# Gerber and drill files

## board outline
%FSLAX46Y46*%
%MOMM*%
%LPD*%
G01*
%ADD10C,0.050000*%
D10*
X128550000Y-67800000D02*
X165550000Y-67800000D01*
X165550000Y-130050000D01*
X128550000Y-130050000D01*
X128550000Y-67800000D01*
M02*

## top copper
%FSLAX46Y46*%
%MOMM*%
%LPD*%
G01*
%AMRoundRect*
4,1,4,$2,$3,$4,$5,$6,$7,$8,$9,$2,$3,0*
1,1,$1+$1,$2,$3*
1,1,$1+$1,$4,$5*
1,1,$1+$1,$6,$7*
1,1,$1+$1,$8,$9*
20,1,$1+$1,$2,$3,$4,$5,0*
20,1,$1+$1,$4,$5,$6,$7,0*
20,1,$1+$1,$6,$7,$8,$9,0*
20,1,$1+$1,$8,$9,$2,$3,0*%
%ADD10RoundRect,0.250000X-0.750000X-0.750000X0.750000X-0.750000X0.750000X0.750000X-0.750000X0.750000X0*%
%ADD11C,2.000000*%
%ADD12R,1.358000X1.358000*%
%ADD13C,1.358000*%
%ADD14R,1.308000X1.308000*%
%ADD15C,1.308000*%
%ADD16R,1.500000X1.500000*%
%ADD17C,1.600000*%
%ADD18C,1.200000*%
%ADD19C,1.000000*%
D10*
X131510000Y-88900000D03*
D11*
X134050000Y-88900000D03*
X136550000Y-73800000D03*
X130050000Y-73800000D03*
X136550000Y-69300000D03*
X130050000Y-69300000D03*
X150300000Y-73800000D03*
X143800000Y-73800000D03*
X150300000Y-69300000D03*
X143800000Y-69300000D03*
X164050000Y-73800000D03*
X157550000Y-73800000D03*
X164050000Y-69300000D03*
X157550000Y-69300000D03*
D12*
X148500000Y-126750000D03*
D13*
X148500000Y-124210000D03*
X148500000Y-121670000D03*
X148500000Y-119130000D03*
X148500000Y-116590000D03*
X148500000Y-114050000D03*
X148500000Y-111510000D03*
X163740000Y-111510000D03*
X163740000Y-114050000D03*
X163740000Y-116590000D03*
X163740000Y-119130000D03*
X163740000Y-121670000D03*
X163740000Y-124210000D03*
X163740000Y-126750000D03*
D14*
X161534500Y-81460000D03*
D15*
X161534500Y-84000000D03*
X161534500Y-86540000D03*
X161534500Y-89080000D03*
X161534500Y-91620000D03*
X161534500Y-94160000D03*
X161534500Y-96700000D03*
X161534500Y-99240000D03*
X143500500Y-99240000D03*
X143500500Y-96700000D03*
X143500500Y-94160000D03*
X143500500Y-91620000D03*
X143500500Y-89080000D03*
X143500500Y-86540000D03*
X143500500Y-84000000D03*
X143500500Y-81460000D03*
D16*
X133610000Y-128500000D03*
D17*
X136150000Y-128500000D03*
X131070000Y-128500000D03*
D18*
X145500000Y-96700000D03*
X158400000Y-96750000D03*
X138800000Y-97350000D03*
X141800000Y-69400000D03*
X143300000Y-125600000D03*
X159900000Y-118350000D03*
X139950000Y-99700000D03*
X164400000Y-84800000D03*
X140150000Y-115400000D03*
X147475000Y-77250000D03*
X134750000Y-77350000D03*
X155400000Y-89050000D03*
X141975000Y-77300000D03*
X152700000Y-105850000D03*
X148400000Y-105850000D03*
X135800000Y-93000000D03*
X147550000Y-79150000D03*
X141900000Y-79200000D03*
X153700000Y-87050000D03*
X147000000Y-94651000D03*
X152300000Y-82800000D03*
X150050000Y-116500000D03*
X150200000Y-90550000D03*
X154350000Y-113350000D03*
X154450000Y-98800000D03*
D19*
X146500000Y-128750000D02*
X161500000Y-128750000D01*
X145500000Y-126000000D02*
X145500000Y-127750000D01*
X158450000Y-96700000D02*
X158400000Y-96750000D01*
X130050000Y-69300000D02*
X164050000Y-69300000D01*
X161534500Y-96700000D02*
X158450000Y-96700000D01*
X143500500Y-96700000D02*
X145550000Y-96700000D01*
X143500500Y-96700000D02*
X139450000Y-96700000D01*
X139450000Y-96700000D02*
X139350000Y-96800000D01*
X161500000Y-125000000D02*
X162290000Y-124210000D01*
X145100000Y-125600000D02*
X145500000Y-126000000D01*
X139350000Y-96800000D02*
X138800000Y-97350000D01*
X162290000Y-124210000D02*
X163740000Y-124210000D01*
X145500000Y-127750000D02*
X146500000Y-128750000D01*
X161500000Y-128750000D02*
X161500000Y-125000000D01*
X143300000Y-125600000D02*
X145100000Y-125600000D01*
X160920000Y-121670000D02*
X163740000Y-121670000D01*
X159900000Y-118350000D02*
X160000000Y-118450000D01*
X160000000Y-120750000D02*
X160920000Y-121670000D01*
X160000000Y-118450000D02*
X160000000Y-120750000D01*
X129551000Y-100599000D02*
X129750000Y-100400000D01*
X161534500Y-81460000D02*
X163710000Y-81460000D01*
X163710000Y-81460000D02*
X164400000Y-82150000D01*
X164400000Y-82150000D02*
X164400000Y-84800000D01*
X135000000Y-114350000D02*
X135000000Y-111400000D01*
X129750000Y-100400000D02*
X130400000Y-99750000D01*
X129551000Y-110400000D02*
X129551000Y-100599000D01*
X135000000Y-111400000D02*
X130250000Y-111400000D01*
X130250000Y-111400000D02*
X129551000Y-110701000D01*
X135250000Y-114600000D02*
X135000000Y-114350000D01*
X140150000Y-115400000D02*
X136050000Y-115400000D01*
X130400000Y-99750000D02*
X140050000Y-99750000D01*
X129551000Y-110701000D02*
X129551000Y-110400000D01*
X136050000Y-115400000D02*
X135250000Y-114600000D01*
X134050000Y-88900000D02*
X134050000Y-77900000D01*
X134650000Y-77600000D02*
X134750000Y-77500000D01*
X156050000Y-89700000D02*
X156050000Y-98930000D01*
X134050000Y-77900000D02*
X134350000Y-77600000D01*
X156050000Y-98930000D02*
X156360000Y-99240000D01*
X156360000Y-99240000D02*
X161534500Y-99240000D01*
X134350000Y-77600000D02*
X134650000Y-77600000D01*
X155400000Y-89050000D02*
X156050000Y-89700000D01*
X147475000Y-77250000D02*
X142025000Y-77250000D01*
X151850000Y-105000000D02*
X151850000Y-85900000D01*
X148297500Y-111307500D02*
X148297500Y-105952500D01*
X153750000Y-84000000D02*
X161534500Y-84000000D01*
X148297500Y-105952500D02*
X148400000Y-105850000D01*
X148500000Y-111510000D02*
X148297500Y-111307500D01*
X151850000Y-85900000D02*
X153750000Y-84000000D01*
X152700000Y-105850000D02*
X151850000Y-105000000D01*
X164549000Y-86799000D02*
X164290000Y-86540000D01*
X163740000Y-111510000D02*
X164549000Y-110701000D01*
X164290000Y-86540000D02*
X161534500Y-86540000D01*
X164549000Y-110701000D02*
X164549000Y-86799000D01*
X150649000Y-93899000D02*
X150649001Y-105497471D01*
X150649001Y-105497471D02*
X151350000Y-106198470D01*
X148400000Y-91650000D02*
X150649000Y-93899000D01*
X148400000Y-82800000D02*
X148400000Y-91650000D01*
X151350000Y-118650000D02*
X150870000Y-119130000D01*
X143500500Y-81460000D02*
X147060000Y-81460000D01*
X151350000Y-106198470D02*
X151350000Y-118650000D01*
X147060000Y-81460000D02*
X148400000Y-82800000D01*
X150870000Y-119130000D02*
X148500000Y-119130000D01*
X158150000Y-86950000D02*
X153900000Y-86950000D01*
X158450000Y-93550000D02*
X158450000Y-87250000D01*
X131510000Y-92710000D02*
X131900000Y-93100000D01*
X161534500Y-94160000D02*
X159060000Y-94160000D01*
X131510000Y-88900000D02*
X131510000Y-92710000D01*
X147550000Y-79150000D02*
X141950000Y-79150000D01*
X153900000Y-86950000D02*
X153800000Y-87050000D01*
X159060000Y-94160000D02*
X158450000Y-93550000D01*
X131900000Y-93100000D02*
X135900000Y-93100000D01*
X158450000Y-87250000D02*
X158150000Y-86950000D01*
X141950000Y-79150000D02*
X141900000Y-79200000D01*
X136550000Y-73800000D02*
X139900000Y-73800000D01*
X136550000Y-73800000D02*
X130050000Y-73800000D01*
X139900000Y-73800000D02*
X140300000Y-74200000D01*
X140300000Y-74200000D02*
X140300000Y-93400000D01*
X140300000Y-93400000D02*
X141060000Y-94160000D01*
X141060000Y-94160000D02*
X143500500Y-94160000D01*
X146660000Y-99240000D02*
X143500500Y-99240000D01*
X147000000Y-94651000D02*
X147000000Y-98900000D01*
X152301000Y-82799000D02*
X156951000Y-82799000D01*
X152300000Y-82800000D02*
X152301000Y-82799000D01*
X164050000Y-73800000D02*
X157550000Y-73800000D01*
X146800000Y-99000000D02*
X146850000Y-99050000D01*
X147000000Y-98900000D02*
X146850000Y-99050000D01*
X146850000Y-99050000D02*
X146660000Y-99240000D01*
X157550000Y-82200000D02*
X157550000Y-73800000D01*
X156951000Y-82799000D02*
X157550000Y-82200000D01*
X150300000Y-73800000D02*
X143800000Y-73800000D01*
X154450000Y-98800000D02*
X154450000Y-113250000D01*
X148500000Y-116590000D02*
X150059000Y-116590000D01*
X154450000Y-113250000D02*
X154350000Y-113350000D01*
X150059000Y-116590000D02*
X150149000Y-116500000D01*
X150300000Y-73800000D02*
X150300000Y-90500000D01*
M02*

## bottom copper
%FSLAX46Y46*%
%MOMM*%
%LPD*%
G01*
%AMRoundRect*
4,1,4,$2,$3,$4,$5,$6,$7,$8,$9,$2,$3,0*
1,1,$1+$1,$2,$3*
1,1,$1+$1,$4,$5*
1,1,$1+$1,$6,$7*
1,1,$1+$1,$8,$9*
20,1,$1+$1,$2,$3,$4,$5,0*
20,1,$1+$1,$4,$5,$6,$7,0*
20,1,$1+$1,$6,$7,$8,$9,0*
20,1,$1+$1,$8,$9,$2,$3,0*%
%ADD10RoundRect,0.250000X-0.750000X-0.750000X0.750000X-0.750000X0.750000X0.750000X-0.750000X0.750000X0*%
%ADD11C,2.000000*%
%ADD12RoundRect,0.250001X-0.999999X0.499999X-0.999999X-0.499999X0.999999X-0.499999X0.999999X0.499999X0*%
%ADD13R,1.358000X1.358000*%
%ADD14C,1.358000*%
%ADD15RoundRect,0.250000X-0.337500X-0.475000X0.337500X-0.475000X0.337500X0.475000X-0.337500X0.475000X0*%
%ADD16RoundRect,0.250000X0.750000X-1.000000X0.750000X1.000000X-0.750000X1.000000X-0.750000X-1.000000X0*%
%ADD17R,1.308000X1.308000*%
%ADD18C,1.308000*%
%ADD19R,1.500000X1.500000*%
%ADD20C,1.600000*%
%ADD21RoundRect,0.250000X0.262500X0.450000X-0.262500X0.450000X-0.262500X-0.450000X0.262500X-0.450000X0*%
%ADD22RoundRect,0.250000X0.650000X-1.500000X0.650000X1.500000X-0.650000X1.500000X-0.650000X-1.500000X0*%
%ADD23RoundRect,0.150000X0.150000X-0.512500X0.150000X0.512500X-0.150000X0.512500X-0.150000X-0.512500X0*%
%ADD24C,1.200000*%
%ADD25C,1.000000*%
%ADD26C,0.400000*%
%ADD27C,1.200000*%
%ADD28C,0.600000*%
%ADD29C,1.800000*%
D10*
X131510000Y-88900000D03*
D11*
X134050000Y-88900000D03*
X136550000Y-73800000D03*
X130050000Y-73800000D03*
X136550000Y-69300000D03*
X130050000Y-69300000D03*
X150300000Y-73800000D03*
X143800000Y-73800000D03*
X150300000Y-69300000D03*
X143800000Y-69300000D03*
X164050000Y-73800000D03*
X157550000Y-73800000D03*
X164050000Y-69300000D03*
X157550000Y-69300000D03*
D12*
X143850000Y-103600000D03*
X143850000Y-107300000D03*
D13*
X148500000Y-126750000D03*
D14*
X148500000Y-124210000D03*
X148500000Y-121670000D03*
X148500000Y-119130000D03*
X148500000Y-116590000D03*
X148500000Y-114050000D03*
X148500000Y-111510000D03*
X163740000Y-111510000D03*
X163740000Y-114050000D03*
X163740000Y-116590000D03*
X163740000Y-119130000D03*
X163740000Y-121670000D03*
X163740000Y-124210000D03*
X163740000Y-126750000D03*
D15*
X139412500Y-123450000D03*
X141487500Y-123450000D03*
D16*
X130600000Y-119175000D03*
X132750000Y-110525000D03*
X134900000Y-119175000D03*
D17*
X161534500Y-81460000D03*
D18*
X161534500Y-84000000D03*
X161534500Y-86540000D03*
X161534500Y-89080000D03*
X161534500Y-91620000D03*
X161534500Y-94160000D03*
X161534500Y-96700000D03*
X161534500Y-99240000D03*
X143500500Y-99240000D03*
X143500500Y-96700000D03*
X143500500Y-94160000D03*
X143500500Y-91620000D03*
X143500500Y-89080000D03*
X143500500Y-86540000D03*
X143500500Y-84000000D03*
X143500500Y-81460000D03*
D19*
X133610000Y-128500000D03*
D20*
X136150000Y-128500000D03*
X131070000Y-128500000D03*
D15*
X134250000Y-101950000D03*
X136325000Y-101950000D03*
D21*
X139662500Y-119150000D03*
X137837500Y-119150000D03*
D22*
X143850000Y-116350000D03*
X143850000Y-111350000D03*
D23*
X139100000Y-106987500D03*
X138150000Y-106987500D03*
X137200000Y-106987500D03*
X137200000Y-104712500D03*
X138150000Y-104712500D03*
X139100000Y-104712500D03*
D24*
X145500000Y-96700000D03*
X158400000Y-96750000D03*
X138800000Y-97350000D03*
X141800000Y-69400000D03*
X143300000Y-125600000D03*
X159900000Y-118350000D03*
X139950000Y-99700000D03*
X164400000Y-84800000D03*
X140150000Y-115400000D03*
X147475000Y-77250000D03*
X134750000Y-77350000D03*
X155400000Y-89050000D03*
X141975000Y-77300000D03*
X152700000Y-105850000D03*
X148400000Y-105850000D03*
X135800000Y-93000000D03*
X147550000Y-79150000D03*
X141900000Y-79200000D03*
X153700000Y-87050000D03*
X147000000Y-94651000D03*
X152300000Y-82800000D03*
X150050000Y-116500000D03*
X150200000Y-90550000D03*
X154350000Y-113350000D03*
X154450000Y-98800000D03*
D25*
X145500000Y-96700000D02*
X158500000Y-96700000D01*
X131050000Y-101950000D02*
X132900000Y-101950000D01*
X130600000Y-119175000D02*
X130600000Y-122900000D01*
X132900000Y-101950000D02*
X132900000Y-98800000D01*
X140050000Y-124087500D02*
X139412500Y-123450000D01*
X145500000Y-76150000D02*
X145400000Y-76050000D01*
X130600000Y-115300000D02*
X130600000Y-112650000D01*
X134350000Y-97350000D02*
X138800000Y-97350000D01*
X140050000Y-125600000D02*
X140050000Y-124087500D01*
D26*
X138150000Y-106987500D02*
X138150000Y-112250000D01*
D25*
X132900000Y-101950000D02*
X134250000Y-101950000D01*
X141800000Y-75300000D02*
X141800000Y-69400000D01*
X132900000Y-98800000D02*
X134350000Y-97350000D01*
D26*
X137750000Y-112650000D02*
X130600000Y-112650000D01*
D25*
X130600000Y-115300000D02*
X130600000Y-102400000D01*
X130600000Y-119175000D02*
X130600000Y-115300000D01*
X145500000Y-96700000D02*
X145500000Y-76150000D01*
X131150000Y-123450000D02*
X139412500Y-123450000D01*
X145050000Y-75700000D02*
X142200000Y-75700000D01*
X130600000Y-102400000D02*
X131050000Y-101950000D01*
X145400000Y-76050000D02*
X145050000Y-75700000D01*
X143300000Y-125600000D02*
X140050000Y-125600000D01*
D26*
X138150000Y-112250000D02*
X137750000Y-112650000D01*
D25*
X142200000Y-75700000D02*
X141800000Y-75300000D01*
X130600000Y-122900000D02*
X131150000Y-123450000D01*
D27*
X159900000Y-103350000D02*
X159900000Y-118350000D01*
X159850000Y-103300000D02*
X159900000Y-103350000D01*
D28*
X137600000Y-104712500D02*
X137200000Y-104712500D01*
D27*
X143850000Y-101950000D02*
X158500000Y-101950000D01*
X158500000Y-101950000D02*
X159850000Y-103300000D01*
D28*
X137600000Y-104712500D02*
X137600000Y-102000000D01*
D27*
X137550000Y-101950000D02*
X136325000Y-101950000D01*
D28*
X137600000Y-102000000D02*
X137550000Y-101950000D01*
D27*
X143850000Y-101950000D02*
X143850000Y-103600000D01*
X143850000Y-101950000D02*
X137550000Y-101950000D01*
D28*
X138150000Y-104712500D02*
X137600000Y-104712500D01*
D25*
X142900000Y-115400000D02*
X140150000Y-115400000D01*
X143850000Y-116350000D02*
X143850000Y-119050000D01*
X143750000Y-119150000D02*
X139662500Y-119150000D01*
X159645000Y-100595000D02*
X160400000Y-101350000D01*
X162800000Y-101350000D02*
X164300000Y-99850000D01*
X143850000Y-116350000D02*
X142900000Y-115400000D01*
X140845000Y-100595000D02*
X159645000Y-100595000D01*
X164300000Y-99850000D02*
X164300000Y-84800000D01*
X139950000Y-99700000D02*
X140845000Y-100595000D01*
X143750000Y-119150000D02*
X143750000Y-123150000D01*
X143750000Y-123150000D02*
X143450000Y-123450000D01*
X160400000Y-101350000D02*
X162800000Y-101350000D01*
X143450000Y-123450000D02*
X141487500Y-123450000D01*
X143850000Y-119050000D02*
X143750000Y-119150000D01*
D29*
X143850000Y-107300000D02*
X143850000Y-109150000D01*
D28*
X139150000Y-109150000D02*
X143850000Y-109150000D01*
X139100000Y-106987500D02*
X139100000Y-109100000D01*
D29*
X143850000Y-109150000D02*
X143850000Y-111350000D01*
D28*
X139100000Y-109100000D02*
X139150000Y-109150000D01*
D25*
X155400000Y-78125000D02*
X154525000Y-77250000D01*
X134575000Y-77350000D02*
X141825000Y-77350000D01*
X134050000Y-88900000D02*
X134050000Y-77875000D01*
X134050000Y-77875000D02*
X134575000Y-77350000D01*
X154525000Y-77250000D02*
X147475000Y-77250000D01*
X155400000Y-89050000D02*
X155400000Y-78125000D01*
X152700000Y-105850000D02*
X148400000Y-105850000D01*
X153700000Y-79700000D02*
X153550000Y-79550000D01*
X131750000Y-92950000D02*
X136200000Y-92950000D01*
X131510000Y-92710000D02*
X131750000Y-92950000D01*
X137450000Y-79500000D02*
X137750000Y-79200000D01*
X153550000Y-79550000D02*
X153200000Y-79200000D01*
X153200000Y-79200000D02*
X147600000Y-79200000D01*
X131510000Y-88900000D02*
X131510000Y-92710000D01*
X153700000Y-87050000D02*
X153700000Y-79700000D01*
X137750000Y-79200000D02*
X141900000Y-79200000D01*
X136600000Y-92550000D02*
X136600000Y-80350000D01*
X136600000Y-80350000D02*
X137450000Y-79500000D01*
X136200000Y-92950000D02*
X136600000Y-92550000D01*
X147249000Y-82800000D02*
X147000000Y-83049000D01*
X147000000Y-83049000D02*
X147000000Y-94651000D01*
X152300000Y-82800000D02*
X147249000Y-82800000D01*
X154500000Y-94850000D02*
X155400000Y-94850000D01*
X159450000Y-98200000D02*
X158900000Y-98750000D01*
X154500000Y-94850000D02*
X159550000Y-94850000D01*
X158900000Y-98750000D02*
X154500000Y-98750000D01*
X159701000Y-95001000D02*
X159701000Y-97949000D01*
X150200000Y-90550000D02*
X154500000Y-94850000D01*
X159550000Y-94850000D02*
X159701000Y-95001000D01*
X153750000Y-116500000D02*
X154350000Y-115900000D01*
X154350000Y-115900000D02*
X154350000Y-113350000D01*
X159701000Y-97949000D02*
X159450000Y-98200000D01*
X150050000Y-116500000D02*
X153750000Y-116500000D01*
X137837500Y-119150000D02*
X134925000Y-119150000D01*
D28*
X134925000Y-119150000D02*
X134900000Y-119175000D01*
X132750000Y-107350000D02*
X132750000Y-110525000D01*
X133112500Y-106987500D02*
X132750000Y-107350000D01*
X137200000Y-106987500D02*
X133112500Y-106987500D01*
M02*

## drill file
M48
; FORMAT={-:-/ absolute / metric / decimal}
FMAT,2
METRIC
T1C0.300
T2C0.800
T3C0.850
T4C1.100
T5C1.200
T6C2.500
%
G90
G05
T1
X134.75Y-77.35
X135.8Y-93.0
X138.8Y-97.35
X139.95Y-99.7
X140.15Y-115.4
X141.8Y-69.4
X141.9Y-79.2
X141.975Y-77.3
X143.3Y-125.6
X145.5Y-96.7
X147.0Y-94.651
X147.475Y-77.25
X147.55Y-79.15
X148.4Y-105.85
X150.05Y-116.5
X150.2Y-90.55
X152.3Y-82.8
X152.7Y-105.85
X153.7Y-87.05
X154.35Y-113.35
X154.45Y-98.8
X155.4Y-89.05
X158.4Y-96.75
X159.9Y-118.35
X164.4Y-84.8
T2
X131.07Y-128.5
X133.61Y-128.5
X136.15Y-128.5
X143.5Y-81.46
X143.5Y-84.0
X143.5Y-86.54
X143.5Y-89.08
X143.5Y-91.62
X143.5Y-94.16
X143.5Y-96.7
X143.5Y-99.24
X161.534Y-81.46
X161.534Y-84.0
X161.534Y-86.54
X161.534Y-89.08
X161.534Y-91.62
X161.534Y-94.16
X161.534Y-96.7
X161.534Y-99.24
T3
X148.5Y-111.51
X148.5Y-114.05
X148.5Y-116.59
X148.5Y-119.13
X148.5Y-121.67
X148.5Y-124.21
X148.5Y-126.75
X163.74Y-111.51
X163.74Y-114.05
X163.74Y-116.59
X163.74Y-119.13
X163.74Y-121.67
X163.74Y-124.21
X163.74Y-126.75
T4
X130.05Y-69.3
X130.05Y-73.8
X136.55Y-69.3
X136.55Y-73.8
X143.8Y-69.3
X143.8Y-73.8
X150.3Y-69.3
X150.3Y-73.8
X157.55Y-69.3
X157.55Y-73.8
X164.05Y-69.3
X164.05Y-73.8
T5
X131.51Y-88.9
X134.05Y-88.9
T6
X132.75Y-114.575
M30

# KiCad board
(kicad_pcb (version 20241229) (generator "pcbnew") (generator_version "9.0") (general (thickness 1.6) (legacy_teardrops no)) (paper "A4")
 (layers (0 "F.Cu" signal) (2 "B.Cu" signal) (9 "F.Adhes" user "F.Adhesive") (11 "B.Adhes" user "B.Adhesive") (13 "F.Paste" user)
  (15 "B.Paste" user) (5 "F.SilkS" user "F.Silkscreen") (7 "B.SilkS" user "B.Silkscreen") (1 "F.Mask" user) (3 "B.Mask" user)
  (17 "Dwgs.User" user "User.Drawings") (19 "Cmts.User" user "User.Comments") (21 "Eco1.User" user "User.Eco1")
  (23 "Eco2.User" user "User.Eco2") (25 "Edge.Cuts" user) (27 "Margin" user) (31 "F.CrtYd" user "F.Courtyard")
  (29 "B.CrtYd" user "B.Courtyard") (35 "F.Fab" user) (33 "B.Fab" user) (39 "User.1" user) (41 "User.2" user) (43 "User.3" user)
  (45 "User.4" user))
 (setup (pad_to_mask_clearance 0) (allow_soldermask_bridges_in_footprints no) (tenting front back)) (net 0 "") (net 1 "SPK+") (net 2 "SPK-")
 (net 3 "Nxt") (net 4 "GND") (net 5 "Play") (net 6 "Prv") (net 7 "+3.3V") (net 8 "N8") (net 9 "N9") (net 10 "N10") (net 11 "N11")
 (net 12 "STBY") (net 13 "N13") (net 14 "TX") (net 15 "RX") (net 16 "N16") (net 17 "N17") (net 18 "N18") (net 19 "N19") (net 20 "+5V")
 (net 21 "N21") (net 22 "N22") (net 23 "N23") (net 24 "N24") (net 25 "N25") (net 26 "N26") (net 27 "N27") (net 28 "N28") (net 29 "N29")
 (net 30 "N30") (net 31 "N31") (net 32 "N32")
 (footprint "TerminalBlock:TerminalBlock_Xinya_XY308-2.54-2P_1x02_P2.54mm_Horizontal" (layer "F.Cu") (at 131.51 88.9)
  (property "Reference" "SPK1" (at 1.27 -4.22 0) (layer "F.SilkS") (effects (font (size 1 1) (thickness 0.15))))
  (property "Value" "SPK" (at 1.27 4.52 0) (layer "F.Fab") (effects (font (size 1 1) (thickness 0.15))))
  (pad "1" thru_hole roundrect (at 0 0) (size 2 2) (drill 1.2) (layers "*.Cu" "*.Mask") (remove_unused_layers no) (roundrect_rratio 0.125)
   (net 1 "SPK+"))
  (pad "2" thru_hole circle (at 2.54 0) (size 2 2) (drill 1.2) (layers "*.Cu" "*.Mask") (remove_unused_layers no) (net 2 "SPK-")))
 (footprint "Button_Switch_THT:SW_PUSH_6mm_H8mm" (layer "F.Cu") (at 136.55 73.8 180)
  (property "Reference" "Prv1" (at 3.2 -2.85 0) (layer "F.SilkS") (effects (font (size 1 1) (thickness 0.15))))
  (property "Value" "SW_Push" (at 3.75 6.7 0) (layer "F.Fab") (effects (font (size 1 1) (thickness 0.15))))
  (pad "1" thru_hole circle (at 0 0 270) (size 2 2) (drill 1.1) (layers "*.Cu" "*.Mask") (remove_unused_layers no) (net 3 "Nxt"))
  (pad "1" thru_hole circle (at 6.5 0 270) (size 2 2) (drill 1.1) (layers "*.Cu" "*.Mask") (remove_unused_layers no) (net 3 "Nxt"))
  (pad "2" thru_hole circle (at 0 4.5 270) (size 2 2) (drill 1.1) (layers "*.Cu" "*.Mask") (remove_unused_layers no) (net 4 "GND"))
  (pad "2" thru_hole circle (at 6.5 4.5 270) (size 2 2) (drill 1.1) (layers "*.Cu" "*.Mask") (remove_unused_layers no) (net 4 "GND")))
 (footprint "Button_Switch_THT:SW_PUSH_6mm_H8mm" (layer "F.Cu") (at 150.3 73.8 180)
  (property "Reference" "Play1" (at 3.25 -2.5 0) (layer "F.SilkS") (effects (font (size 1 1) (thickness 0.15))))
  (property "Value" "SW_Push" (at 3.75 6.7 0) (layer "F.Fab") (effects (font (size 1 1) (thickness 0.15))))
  (pad "1" thru_hole circle (at 0 0 270) (size 2 2) (drill 1.1) (layers "*.Cu" "*.Mask") (remove_unused_layers no) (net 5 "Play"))
  (pad "1" thru_hole circle (at 6.5 0 270) (size 2 2) (drill 1.1) (layers "*.Cu" "*.Mask") (remove_unused_layers no) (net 5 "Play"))
  (pad "2" thru_hole circle (at 0 4.5 270) (size 2 2) (drill 1.1) (layers "*.Cu" "*.Mask") (remove_unused_layers no) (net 4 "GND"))
  (pad "2" thru_hole circle (at 6.5 4.5 270) (size 2 2) (drill 1.1) (layers "*.Cu" "*.Mask") (remove_unused_layers no) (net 4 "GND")))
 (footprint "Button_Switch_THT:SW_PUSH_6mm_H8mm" (layer "F.Cu") (at 164.05 73.8 180)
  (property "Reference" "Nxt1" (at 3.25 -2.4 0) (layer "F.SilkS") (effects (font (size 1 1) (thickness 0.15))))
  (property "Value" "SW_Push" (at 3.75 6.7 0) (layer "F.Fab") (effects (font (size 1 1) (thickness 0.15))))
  (pad "1" thru_hole circle (at 0 0 270) (size 2 2) (drill 1.1) (layers "*.Cu" "*.Mask") (remove_unused_layers no) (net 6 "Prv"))
  (pad "1" thru_hole circle (at 6.5 0 270) (size 2 2) (drill 1.1) (layers "*.Cu" "*.Mask") (remove_unused_layers no) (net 6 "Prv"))
  (pad "2" thru_hole circle (at 0 4.5 270) (size 2 2) (drill 1.1) (layers "*.Cu" "*.Mask") (remove_unused_layers no) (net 4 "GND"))
  (pad "2" thru_hole circle (at 6.5 4.5 270) (size 2 2) (drill 1.1) (layers "*.Cu" "*.Mask") (remove_unused_layers no) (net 4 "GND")))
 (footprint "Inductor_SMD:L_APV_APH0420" (layer "B.Cu") (at 143.85 105.45 -90)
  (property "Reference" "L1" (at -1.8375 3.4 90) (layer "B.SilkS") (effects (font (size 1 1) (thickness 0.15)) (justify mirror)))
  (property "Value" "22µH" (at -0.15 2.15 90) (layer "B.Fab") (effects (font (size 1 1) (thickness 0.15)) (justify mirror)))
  (pad "1" smd roundrect (at -1.85 0 270) (size 1.5 2.5) (layers "B.Cu" "B.Mask" "B.Paste") (roundrect_rratio 0.166667) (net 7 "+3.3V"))
  (pad "2" smd roundrect (at 1.85 0 270) (size 1.5 2.5) (layers "B.Cu" "B.Mask" "B.Paste") (roundrect_rratio 0.166667) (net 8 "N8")))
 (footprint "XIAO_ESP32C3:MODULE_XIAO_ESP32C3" (layer "B.Cu") (at 156.12 119.1935)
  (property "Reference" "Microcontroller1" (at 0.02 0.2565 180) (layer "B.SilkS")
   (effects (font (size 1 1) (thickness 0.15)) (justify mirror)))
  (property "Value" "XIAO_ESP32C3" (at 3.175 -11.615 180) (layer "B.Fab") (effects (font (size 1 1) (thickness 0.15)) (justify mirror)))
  (pad "1" thru_hole rect (at -7.62 7.5565) (size 1.358 1.358) (drill 0.85) (layers "*.Cu" "*.Mask") (remove_unused_layers no) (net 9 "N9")
   (solder_mask_margin 0.102))
  (pad "2" thru_hole circle (at -7.62 5.0165) (size 1.358 1.358) (drill 0.85) (layers "*.Cu" "*.Mask") (remove_unused_layers no)
   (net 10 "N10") (solder_mask_margin 0.102))
  (pad "3" thru_hole circle (at -7.62 2.4765) (size 1.358 1.358) (drill 0.85) (layers "*.Cu" "*.Mask") (remove_unused_layers no)
   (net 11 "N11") (solder_mask_margin 0.102))
  (pad "4" thru_hole circle (at -7.62 -0.0635) (size 1.358 1.358) (drill 0.85) (layers "*.Cu" "*.Mask") (remove_unused_layers no)
   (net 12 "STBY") (solder_mask_margin 0.102))
  (pad "5" thru_hole circle (at -7.62 -2.6035) (size 1.358 1.358) (drill 0.85) (layers "*.Cu" "*.Mask") (remove_unused_layers no)
   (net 5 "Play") (solder_mask_margin 0.102))
  (pad "6" thru_hole circle (at -7.62 -5.1435) (size 1.358 1.358) (drill 0.85) (layers "*.Cu" "*.Mask") (remove_unused_layers no)
   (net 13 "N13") (solder_mask_margin 0.102))
  (pad "7" thru_hole circle (at -7.62 -7.6835) (size 1.358 1.358) (drill 0.85) (layers "*.Cu" "*.Mask") (remove_unused_layers no)
   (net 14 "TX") (solder_mask_margin 0.102))
  (pad "8" thru_hole circle (at 7.62 -7.6835) (size 1.358 1.358) (drill 0.85) (layers "*.Cu" "*.Mask") (remove_unused_layers no)
   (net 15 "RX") (solder_mask_margin 0.102))
  (pad "9" thru_hole circle (at 7.62 -5.1435) (size 1.358 1.358) (drill 0.85) (layers "*.Cu" "*.Mask") (remove_unused_layers no)
   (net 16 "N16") (solder_mask_margin 0.102))
  (pad "10" thru_hole circle (at 7.62 -2.6035) (size 1.358 1.358) (drill 0.85) (layers "*.Cu" "*.Mask") (remove_unused_layers no)
   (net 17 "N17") (solder_mask_margin 0.102))
  (pad "11" thru_hole circle (at 7.62 -0.0635) (size 1.358 1.358) (drill 0.85) (layers "*.Cu" "*.Mask") (remove_unused_layers no)
   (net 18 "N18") (solder_mask_margin 0.102))
  (pad "12" thru_hole circle (at 7.62 2.4765) (size 1.358 1.358) (drill 0.85) (layers "*.Cu" "*.Mask") (remove_unused_layers no)
   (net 7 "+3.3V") (solder_mask_margin 0.102))
  (pad "13" thru_hole circle (at 7.62 5.0165) (size 1.358 1.358) (drill 0.85) (layers "*.Cu" "*.Mask") (remove_unused_layers no)
   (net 4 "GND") (solder_mask_margin 0.102))
  (pad "14" thru_hole circle (at 7.62 7.5565) (size 1.358 1.358) (drill 0.85) (layers "*.Cu" "*.Mask") (remove_unused_layers no)
   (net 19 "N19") (solder_mask_margin 0.102)))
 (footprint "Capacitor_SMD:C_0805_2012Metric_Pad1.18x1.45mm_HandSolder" (layer "B.Cu") (at 140.45 123.45)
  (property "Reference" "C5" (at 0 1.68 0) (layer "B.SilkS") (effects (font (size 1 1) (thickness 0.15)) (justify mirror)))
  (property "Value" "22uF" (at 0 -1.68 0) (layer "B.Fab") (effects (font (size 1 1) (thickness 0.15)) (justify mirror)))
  (pad "1" smd roundrect (at -1.0375 0) (size 1.175 1.45) (layers "B.Cu" "B.Mask" "B.Paste") (roundrect_rratio 0.212766) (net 4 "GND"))
  (pad "2" smd roundrect (at 1.0375 0) (size 1.175 1.45) (layers "B.Cu" "B.Mask" "B.Paste") (roundrect_rratio 0.212766) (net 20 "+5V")))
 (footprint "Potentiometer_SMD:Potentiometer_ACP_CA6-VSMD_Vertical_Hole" (layer "B.Cu") (at 132.75 114.85 90)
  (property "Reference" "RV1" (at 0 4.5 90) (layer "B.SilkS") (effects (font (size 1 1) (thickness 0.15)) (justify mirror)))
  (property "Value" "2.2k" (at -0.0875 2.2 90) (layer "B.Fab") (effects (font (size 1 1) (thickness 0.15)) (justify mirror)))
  (pad "" np_thru_hole circle (at 0.275 0 90) (size 2.5 2.5) (drill 2.5) (layers "*.Cu" "*.Mask"))
  (pad "1" smd roundrect (at -4.325 -2.15 90) (size 2.5 2) (layers "B.Cu" "B.Mask" "B.Paste") (roundrect_rratio 0.125) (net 4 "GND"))
  (pad "2" smd roundrect (at 4.325 0 90) (size 2.5 2) (layers "B.Cu" "B.Mask" "B.Paste") (roundrect_rratio 0.125) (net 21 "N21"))
  (pad "3" smd roundrect (at -4.325 2.15 90) (size 2.5 2) (layers "B.Cu" "B.Mask" "B.Paste") (roundrect_rratio 0.125) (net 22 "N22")))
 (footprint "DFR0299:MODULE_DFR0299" (layer "B.Cu") (at 152.5175 90.35 180)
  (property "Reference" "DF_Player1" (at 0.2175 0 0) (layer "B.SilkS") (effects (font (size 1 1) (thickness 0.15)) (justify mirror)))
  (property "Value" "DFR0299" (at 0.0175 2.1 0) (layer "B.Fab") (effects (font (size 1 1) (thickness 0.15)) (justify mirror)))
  (pad "1" thru_hole rect (at -9.017 8.89 180) (size 1.308 1.308) (drill 0.8) (layers "*.Cu" "*.Mask") (remove_unused_layers no)
   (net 20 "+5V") (solder_mask_margin 0.102))
  (pad "2" thru_hole circle (at -9.017 6.35 180) (size 1.308 1.308) (drill 0.8) (layers "*.Cu" "*.Mask") (remove_unused_layers no)
   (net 14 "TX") (solder_mask_margin 0.102))
  (pad "3" thru_hole circle (at -9.017 3.81 180) (size 1.308 1.308) (drill 0.8) (layers "*.Cu" "*.Mask") (remove_unused_layers no)
   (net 15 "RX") (solder_mask_margin 0.102))
  (pad "4" thru_hole circle (at -9.017 1.27 180) (size 1.308 1.308) (drill 0.8) (layers "*.Cu" "*.Mask") (remove_unused_layers no)
   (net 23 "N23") (solder_mask_margin 0.102))
  (pad "5" thru_hole circle (at -9.017 -1.27 180) (size 1.308 1.308) (drill 0.8) (layers "*.Cu" "*.Mask") (remove_unused_layers no)
   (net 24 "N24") (solder_mask_margin 0.102))
  (pad "6" thru_hole circle (at -9.017 -3.81 180) (size 1.308 1.308) (drill 0.8) (layers "*.Cu" "*.Mask") (remove_unused_layers no)
   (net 1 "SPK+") (solder_mask_margin 0.102))
  (pad "7" thru_hole circle (at -9.017 -6.35 180) (size 1.308 1.308) (drill 0.8) (layers "*.Cu" "*.Mask") (remove_unused_layers no)
   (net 4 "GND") (solder_mask_margin 0.102))
  (pad "8" thru_hole circle (at -9.017 -8.89 180) (size 1.308 1.308) (drill 0.8) (layers "*.Cu" "*.Mask") (remove_unused_layers no)
   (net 2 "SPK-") (solder_mask_margin 0.102))
  (pad "9" thru_hole circle (at 9.017 -8.89 180) (size 1.308 1.308) (drill 0.8) (layers "*.Cu" "*.Mask") (remove_unused_layers no)
   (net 6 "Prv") (solder_mask_margin 0.102))
  (pad "10" thru_hole circle (at 9.017 -6.35 180) (size 1.308 1.308) (drill 0.8) (layers "*.Cu" "*.Mask") (remove_unused_layers no)
   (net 4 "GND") (solder_mask_margin 0.102))
  (pad "11" thru_hole circle (at 9.017 -3.81 180) (size 1.308 1.308) (drill 0.8) (layers "*.Cu" "*.Mask") (remove_unused_layers no)
   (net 3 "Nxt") (solder_mask_margin 0.102))
  (pad "12" thru_hole circle (at 9.017 -1.27 180) (size 1.308 1.308) (drill 0.8) (layers "*.Cu" "*.Mask") (remove_unused_layers no)
   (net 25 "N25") (solder_mask_margin 0.102))
  (pad "13" thru_hole circle (at 9.017 1.27 180) (size 1.308 1.308) (drill 0.8) (layers "*.Cu" "*.Mask") (remove_unused_layers no)
   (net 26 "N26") (solder_mask_margin 0.102))
  (pad "14" thru_hole circle (at 9.017 3.81 180) (size 1.308 1.308) (drill 0.8) (layers "*.Cu" "*.Mask") (remove_unused_layers no)
   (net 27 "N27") (solder_mask_margin 0.102))
  (pad "15" thru_hole circle (at 9.017 6.35 180) (size 1.308 1.308) (drill 0.8) (layers "*.Cu" "*.Mask") (remove_unused_layers no)
   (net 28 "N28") (solder_mask_margin 0.102))
  (pad "16" thru_hole circle (at 9.017 8.89 180) (size 1.308 1.308) (drill 0.8) (layers "*.Cu" "*.Mask") (remove_unused_layers no)
   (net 12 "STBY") (solder_mask_margin 0.102)))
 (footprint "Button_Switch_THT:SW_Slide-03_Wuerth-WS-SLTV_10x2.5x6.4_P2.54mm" (layer "B.Cu") (at 133.61 128.5 180)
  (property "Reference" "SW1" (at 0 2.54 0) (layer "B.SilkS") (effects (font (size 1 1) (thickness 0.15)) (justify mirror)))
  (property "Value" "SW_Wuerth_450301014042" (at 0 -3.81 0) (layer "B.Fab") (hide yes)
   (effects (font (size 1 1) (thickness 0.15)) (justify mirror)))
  (pad "1" thru_hole rect (at 0 0 180) (size 1.5 1.5) (drill 0.8) (layers "*.Cu" "*.Mask") (remove_unused_layers no) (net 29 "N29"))
  (pad "2" thru_hole circle (at -2.54 0 180) (size 1.6 1.6) (drill 0.8) (layers "*.Cu" "*.Mask") (remove_unused_layers no) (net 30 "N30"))
  (pad "3" thru_hole circle (at 2.54 0 180) (size 1.6 1.6) (drill 0.8) (layers "*.Cu" "*.Mask") (remove_unused_layers no) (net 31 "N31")))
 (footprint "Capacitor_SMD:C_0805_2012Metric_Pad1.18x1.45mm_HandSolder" (layer "B.Cu") (at 135.2875 101.95)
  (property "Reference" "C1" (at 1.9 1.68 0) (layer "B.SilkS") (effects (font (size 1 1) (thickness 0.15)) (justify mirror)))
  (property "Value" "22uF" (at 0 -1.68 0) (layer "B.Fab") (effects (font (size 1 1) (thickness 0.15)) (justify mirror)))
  (pad "1" smd roundrect (at -1.0375 0) (size 1.175 1.45) (layers "B.Cu" "B.Mask" "B.Paste") (roundrect_rratio 0.212766) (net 4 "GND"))
  (pad "2" smd roundrect (at 1.0375 0) (size 1.175 1.45) (layers "B.Cu" "B.Mask" "B.Paste") (roundrect_rratio 0.212766) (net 7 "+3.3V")))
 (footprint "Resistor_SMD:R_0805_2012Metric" (layer "B.Cu") (at 138.75 119.15 180)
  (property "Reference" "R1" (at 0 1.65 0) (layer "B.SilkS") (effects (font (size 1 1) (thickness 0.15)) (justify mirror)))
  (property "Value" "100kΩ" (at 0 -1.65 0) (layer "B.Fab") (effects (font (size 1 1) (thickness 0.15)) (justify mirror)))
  (pad "1" smd roundrect (at -0.9125 0 180) (size 1.025 1.4) (layers "B.Cu" "B.Mask" "B.Paste") (roundrect_rratio 0.243902) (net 20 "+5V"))
  (pad "2" smd roundrect (at 0.9125 0 180) (size 1.025 1.4) (layers "B.Cu" "B.Mask" "B.Paste") (roundrect_rratio 0.243902) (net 22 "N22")))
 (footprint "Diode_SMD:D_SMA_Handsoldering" (layer "B.Cu") (at 143.85 113.85 90)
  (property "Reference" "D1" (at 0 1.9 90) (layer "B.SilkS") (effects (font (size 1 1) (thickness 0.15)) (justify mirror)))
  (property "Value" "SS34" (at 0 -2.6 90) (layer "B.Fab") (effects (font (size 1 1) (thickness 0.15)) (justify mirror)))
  (pad "1" smd roundrect (at -2.5 0 90) (size 3.5 1.8) (layers "B.Cu" "B.Mask" "B.Paste") (roundrect_rratio 0.1388888889) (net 20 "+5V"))
  (pad "2" smd roundrect (at 2.5 0 90) (size 3.5 1.8) (layers "B.Cu" "B.Mask" "B.Paste") (roundrect_rratio 0.1388888889) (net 8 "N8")))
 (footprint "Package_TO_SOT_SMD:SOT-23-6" (layer "B.Cu") (at 138.15 105.85 90)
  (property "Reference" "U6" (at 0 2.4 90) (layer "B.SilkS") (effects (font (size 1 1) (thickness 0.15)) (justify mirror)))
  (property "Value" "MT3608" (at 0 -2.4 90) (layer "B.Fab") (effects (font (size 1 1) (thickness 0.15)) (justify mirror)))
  (pad "1" smd roundrect (at -1.1375 0.95 90) (size 1.325 0.6) (layers "B.Cu" "B.Mask" "B.Paste") (roundrect_rratio 0.25) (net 8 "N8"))
  (pad "2" smd roundrect (at -1.1375 0 90) (size 1.325 0.6) (layers "B.Cu" "B.Mask" "B.Paste") (roundrect_rratio 0.25) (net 4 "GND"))
  (pad "3" smd roundrect (at -1.1375 -0.95 90) (size 1.325 0.6) (layers "B.Cu" "B.Mask" "B.Paste") (roundrect_rratio 0.25) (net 21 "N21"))
  (pad "4" smd roundrect (at 1.1375 -0.95 90) (size 1.325 0.6) (layers "B.Cu" "B.Mask" "B.Paste") (roundrect_rratio 0.25) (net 7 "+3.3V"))
  (pad "5" smd roundrect (at 1.1375 0 90) (size 1.325 0.6) (layers "B.Cu" "B.Mask" "B.Paste") (roundrect_rratio 0.25) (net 7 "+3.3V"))
  (pad "6" smd roundrect (at 1.1375 0.95 90) (size 1.325 0.6) (layers "B.Cu" "B.Mask" "B.Paste") (roundrect_rratio 0.25) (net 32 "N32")))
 (gr_rect (start 128.55 67.8) (end 165.55 130.05) (stroke (width 0.05) (type solid)) (fill no) (layer "Edge.Cuts"))
 (segment (start 146.5 128.75) (end 161.5 128.75) (width 1) (layer "F.Cu") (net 4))
 (segment (start 145.5 126) (end 145.5 127.75) (width 1) (layer "F.Cu") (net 4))
 (segment (start 158.45 96.7) (end 158.4 96.75) (width 1) (layer "F.Cu") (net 4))
 (segment (start 130.05 69.3) (end 164.05 69.3) (width 1) (layer "F.Cu") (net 4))
 (segment (start 161.5345 96.7) (end 158.45 96.7) (width 1) (layer "F.Cu") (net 4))
 (segment (start 143.5005 96.7) (end 145.55 96.7) (width 1) (layer "F.Cu") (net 4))
 (segment (start 143.5005 96.7) (end 139.45 96.7) (width 1) (layer "F.Cu") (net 4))
 (segment (start 139.45 96.7) (end 139.35 96.8) (width 1) (layer "F.Cu") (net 4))
 (segment (start 161.5 125) (end 162.29 124.21) (width 1) (layer "F.Cu") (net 4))
 (segment (start 145.1 125.6) (end 145.5 126) (width 1) (layer "F.Cu") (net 4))
 (segment (start 139.35 96.8) (end 138.8 97.35) (width 1) (layer "F.Cu") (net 4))
 (segment (start 162.29 124.21) (end 163.74 124.21) (width 1) (layer "F.Cu") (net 4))
 (segment (start 145.5 127.75) (end 146.5 128.75) (width 1) (layer "F.Cu") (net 4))
 (segment (start 161.5 128.75) (end 161.5 125) (width 1) (layer "F.Cu") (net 4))
 (segment (start 143.3 125.6) (end 145.1 125.6) (width 1) (layer "F.Cu") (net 4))
 (via (at 145.5 96.7) (size 1.2) (drill 0.3) (layers "F.Cu" "B.Cu") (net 4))
 (via (at 158.4 96.75) (size 1.2) (drill 0.3) (layers "F.Cu" "B.Cu") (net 4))
 (via (at 138.8 97.35) (size 1.2) (drill 0.3) (layers "F.Cu" "B.Cu") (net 4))
 (via (at 141.8 69.4) (size 1.2) (drill 0.3) (layers "F.Cu" "B.Cu") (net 4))
 (via (at 143.3 125.6) (size 1.2) (drill 0.3) (layers "F.Cu" "B.Cu") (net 4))
 (segment (start 145.5 96.7) (end 158.5 96.7) (width 1) (layer "B.Cu") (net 4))
 (segment (start 131.05 101.95) (end 132.9 101.95) (width 1) (layer "B.Cu") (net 4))
 (segment (start 130.6 119.175) (end 130.6 122.9) (width 1) (layer "B.Cu") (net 4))
 (segment (start 132.9 101.95) (end 132.9 98.8) (width 1) (layer "B.Cu") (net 4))
 (segment (start 140.05 124.0875) (end 139.4125 123.45) (width 1) (layer "B.Cu") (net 4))
 (segment (start 145.5 76.15) (end 145.4 76.05) (width 1) (layer "B.Cu") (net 4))
 (segment (start 130.6 115.3) (end 130.6 112.65) (width 1) (layer "B.Cu") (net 4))
 (segment (start 134.35 97.35) (end 138.8 97.35) (width 1) (layer "B.Cu") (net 4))
 (segment (start 140.05 125.6) (end 140.05 124.0875) (width 1) (layer "B.Cu") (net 4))
 (segment (start 138.15 106.9875) (end 138.15 112.25) (width 0.4) (layer "B.Cu") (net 4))
 (segment (start 132.9 101.95) (end 134.25 101.95) (width 1) (layer "B.Cu") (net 4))
 (segment (start 141.8 75.3) (end 141.8 69.4) (width 1) (layer "B.Cu") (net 4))
 (segment (start 132.9 98.8) (end 134.35 97.35) (width 1) (layer "B.Cu") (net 4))
 (segment (start 137.75 112.65) (end 130.6 112.65) (width 0.4) (layer "B.Cu") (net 4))
 (segment (start 130.6 115.3) (end 130.6 102.4) (width 1) (layer "B.Cu") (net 4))
 (segment (start 130.6 119.175) (end 130.6 115.3) (width 1) (layer "B.Cu") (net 4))
 (segment (start 145.5 96.7) (end 145.5 76.15) (width 1) (layer "B.Cu") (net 4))
 (segment (start 131.15 123.45) (end 139.4125 123.45) (width 1) (layer "B.Cu") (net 4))
 (segment (start 145.05 75.7) (end 142.2 75.7) (width 1) (layer "B.Cu") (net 4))
 (segment (start 130.6 102.4) (end 131.05 101.95) (width 1) (layer "B.Cu") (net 4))
 (segment (start 145.4 76.05) (end 145.05 75.7) (width 1) (layer "B.Cu") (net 4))
 (segment (start 143.3 125.6) (end 140.05 125.6) (width 1) (layer "B.Cu") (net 4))
 (segment (start 138.15 112.25) (end 137.75 112.65) (width 0.4) (layer "B.Cu") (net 4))
 (segment (start 142.2 75.7) (end 141.8 75.3) (width 1) (layer "B.Cu") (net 4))
 (segment (start 130.6 122.9) (end 131.15 123.45) (width 1) (layer "B.Cu") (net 4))
 (segment (start 160.92 121.67) (end 163.74 121.67) (width 1) (layer "F.Cu") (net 7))
 (segment (start 159.9 118.35) (end 160 118.45) (width 1) (layer "F.Cu") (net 7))
 (segment (start 160 120.75) (end 160.92 121.67) (width 1) (layer "F.Cu") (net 7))
 (segment (start 160 118.45) (end 160 120.75) (width 1) (layer "F.Cu") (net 7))
 (via (at 159.9 118.35) (size 1.2) (drill 0.3) (layers "F.Cu" "B.Cu") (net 7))
 (segment (start 159.9 103.35) (end 159.9 118.35) (width 1.2) (layer "B.Cu") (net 7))
 (segment (start 159.85 103.3) (end 159.9 103.35) (width 1.2) (layer "B.Cu") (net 7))
 (segment (start 137.6 104.7125) (end 137.2 104.7125) (width 0.6) (layer "B.Cu") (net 7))
 (segment (start 143.85 101.95) (end 158.5 101.95) (width 1.2) (layer "B.Cu") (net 7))
 (segment (start 158.5 101.95) (end 159.85 103.3) (width 1.2) (layer "B.Cu") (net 7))
 (segment (start 137.6 104.7125) (end 137.6 102) (width 0.6) (layer "B.Cu") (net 7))
 (segment (start 137.55 101.95) (end 136.325 101.95) (width 1.2) (layer "B.Cu") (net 7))
 (segment (start 137.6 102) (end 137.55 101.95) (width 0.6) (layer "B.Cu") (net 7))
 (segment (start 143.85 101.95) (end 143.85 103.6) (width 1.2) (layer "B.Cu") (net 7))
 (segment (start 143.85 101.95) (end 137.55 101.95) (width 1.2) (layer "B.Cu") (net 7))
 (segment (start 138.15 104.7125) (end 137.6 104.7125) (width 0.6) (layer "B.Cu") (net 7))
 (segment (start 129.551 100.599) (end 129.75 100.4) (width 1) (layer "F.Cu") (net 20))
 (segment (start 161.5345 81.46) (end 163.71 81.46) (width 1) (layer "F.Cu") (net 20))
 (segment (start 163.71 81.46) (end 164.4 82.15) (width 1) (layer "F.Cu") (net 20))
 (segment (start 164.4 82.15) (end 164.4 84.8) (width 1) (layer "F.Cu") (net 20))
 (segment (start 135 114.35) (end 135 111.4) (width 1) (layer "F.Cu") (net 20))
 (segment (start 129.75 100.4) (end 130.4 99.75) (width 1) (layer "F.Cu") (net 20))
 (segment (start 129.551 110.4) (end 129.551 100.599) (width 1) (layer "F.Cu") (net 20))
 (segment (start 135 111.4) (end 130.25 111.4) (width 1) (layer "F.Cu") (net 20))
 (segment (start 130.25 111.4) (end 129.551 110.701) (width 1) (layer "F.Cu") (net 20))
 (segment (start 135.25 114.6) (end 135 114.35) (width 1) (layer "F.Cu") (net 20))
 (segment (start 140.15 115.4) (end 136.05 115.4) (width 1) (layer "F.Cu") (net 20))
 (segment (start 130.4 99.75) (end 140.05 99.75) (width 1) (layer "F.Cu") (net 20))
 (segment (start 129.551 110.701) (end 129.551 110.4) (width 1) (layer "F.Cu") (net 20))
 (segment (start 136.05 115.4) (end 135.25 114.6) (width 1) (layer "F.Cu") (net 20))
 (via (at 139.95 99.7) (size 1.2) (drill 0.3) (layers "F.Cu" "B.Cu") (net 20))
 (via (at 164.4 84.8) (size 1.2) (drill 0.3) (layers "F.Cu" "B.Cu") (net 20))
 (via (at 140.15 115.4) (size 1.2) (drill 0.3) (layers "F.Cu" "B.Cu") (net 20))
 (segment (start 142.9 115.4) (end 140.15 115.4) (width 1) (layer "B.Cu") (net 20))
 (segment (start 143.85 116.35) (end 143.85 119.05) (width 1) (layer "B.Cu") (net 20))
 (segment (start 143.75 119.15) (end 139.6625 119.15) (width 1) (layer "B.Cu") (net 20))
 (segment (start 159.645 100.595) (end 160.4 101.35) (width 1) (layer "B.Cu") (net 20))
 (segment (start 162.8 101.35) (end 164.3 99.85) (width 1) (layer "B.Cu") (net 20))
 (segment (start 143.85 116.35) (end 142.9 115.4) (width 1) (layer "B.Cu") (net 20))
 (segment (start 140.845 100.595) (end 159.645 100.595) (width 1) (layer "B.Cu") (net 20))
 (segment (start 164.3 99.85) (end 164.3 84.8) (width 1) (layer "B.Cu") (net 20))
 (segment (start 139.95 99.7) (end 140.845 100.595) (width 1) (layer "B.Cu") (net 20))
 (segment (start 143.75 119.15) (end 143.75 123.15) (width 1) (layer "B.Cu") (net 20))
 (segment (start 143.75 123.15) (end 143.45 123.45) (width 1) (layer "B.Cu") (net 20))
 (segment (start 160.4 101.35) (end 162.8 101.35) (width 1) (layer "B.Cu") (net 20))
 (segment (start 143.45 123.45) (end 141.4875 123.45) (width 1) (layer "B.Cu") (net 20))
 (segment (start 143.85 119.05) (end 143.75 119.15) (width 1) (layer "B.Cu") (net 20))
 (segment (start 143.85 107.3) (end 143.85 109.15) (width 1.8) (layer "B.Cu") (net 8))
 (segment (start 139.15 109.15) (end 143.85 109.15) (width 0.6) (layer "B.Cu") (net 8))
 (segment (start 139.1 106.9875) (end 139.1 109.1) (width 0.6) (layer "B.Cu") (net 8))
 (segment (start 143.85 109.15) (end 143.85 111.35) (width 1.8) (layer "B.Cu") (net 8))
 (segment (start 139.1 109.1) (end 139.15 109.15) (width 0.6) (layer "B.Cu") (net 8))
 (segment (start 134.05 88.9) (end 134.05 77.9) (width 1) (layer "F.Cu") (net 2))
 (segment (start 134.65 77.6) (end 134.75 77.5) (width 1) (layer "F.Cu") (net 2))
 (segment (start 156.05 89.7) (end 156.05 98.93) (width 1) (layer "F.Cu") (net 2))
 (segment (start 134.05 77.9) (end 134.35 77.6) (width 1) (layer "F.Cu") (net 2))
 (segment (start 156.05 98.93) (end 156.36 99.24) (width 1) (layer "F.Cu") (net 2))
 (segment (start 156.36 99.24) (end 161.5345 99.24) (width 1) (layer "F.Cu") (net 2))
 (segment (start 134.35 77.6) (end 134.65 77.6) (width 1) (layer "F.Cu") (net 2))
 (segment (start 155.4 89.05) (end 156.05 89.7) (width 1) (layer "F.Cu") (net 2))
 (segment (start 147.475 77.25) (end 142.025 77.25) (width 1) (layer "F.Cu") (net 2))
 (via (at 147.475 77.25) (size 1.2) (drill 0.3) (layers "F.Cu" "B.Cu") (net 2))
 (via (at 134.75 77.35) (size 1.2) (drill 0.3) (layers "F.Cu" "B.Cu") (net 2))
 (via (at 155.4 89.05) (size 1.2) (drill 0.3) (layers "F.Cu" "B.Cu") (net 2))
 (via (at 141.975 77.3) (size 1.2) (drill 0.3) (layers "F.Cu" "B.Cu") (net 2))
 (segment (start 155.4 78.125) (end 154.525 77.25) (width 1) (layer "B.Cu") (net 2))
 (segment (start 134.575 77.35) (end 141.825 77.35) (width 1) (layer "B.Cu") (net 2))
 (segment (start 134.05 88.9) (end 134.05 77.875) (width 1) (layer "B.Cu") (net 2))
 (segment (start 134.05 77.875) (end 134.575 77.35) (width 1) (layer "B.Cu") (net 2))
 (segment (start 154.525 77.25) (end 147.475 77.25) (width 1) (layer "B.Cu") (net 2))
 (segment (start 155.4 89.05) (end 155.4 78.125) (width 1) (layer "B.Cu") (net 2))
 (segment (start 151.85 105) (end 151.85 85.9) (width 1) (layer "F.Cu") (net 14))
 (segment (start 148.2975 111.3075) (end 148.2975 105.9525) (width 1) (layer "F.Cu") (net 14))
 (segment (start 153.75 84) (end 161.5345 84) (width 1) (layer "F.Cu") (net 14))
 (segment (start 148.2975 105.9525) (end 148.4 105.85) (width 1) (layer "F.Cu") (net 14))
 (segment (start 148.5 111.51) (end 148.2975 111.3075) (width 1) (layer "F.Cu") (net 14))
 (segment (start 151.85 85.9) (end 153.75 84) (width 1) (layer "F.Cu") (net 14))
 (segment (start 152.7 105.85) (end 151.85 105) (width 1) (layer "F.Cu") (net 14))
 (via (at 152.7 105.85) (size 1.2) (drill 0.3) (layers "F.Cu" "B.Cu") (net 14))
 (via (at 148.4 105.85) (size 1.2) (drill 0.3) (layers "F.Cu" "B.Cu") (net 14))
 (segment (start 152.7 105.85) (end 148.4 105.85) (width 1) (layer "B.Cu") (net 14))
 (segment (start 164.549 86.799) (end 164.29 86.54) (width 1) (layer "F.Cu") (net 15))
 (segment (start 163.74 111.51) (end 164.549 110.701) (width 1) (layer "F.Cu") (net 15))
 (segment (start 164.29 86.54) (end 161.5345 86.54) (width 1) (layer "F.Cu") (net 15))
 (segment (start 164.549 110.701) (end 164.549 86.799) (width 1) (layer "F.Cu") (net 15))
 (segment (start 150.649 93.899) (end 150.649001 105.497471) (width 1) (layer "F.Cu") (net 12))
 (segment (start 150.649001 105.497471) (end 151.35 106.19847) (width 1) (layer "F.Cu") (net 12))
 (segment (start 148.4 91.65) (end 150.649 93.899) (width 1) (layer "F.Cu") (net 12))
 (segment (start 148.4 82.8) (end 148.4 91.65) (width 1) (layer "F.Cu") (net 12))
 (segment (start 151.35 118.65) (end 150.87 119.13) (width 1) (layer "F.Cu") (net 12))
 (segment (start 143.5005 81.46) (end 147.06 81.46) (width 1) (layer "F.Cu") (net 12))
 (segment (start 151.35 106.19847) (end 151.35 118.65) (width 1) (layer "F.Cu") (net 12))
 (segment (start 147.06 81.46) (end 148.4 82.8) (width 1) (layer "F.Cu") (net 12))
 (segment (start 150.87 119.13) (end 148.5 119.13) (width 1) (layer "F.Cu") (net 12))
 (segment (start 158.15 86.95) (end 153.9 86.95) (width 1) (layer "F.Cu") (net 1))
 (segment (start 158.45 93.55) (end 158.45 87.25) (width 1) (layer "F.Cu") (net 1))
 (segment (start 131.51 92.71) (end 131.9 93.1) (width 1) (layer "F.Cu") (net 1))
 (segment (start 161.5345 94.16) (end 159.06 94.16) (width 1) (layer "F.Cu") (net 1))
 (segment (start 131.51 88.9) (end 131.51 92.71) (width 1) (layer "F.Cu") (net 1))
 (segment (start 147.55 79.15) (end 141.95 79.15) (width 1) (layer "F.Cu") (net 1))
 (segment (start 153.9 86.95) (end 153.8 87.05) (width 1) (layer "F.Cu") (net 1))
 (segment (start 159.06 94.16) (end 158.45 93.55) (width 1) (layer "F.Cu") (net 1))
 (segment (start 131.9 93.1) (end 135.9 93.1) (width 1) (layer "F.Cu") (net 1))
 (segment (start 158.45 87.25) (end 158.15 86.95) (width 1) (layer "F.Cu") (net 1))
 (segment (start 141.95 79.15) (end 141.9 79.2) (width 1) (layer "F.Cu") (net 1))
 (via (at 135.8 93) (size 1.2) (drill 0.3) (layers "F.Cu" "B.Cu") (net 1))
 (via (at 147.55 79.15) (size 1.2) (drill 0.3) (layers "F.Cu" "B.Cu") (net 1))
 (via (at 141.9 79.2) (size 1.2) (drill 0.3) (layers "F.Cu" "B.Cu") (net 1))
 (via (at 153.7 87.05) (size 1.2) (drill 0.3) (layers "F.Cu" "B.Cu") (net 1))
 (segment (start 153.7 79.7) (end 153.55 79.55) (width 1) (layer "B.Cu") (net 1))
 (segment (start 131.75 92.95) (end 136.2 92.95) (width 1) (layer "B.Cu") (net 1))
 (segment (start 131.51 92.71) (end 131.75 92.95) (width 1) (layer "B.Cu") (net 1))
 (segment (start 137.45 79.5) (end 137.75 79.2) (width 1) (layer "B.Cu") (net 1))
 (segment (start 153.55 79.55) (end 153.2 79.2) (width 1) (layer "B.Cu") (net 1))
 (segment (start 153.2 79.2) (end 147.6 79.2) (width 1) (layer "B.Cu") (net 1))
 (segment (start 131.51 88.9) (end 131.51 92.71) (width 1) (layer "B.Cu") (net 1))
 (segment (start 153.7 87.05) (end 153.7 79.7) (width 1) (layer "B.Cu") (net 1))
 (segment (start 137.75 79.2) (end 141.9 79.2) (width 1) (layer "B.Cu") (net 1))
 (segment (start 136.6 92.55) (end 136.6 80.35) (width 1) (layer "B.Cu") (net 1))
 (segment (start 136.6 80.35) (end 137.45 79.5) (width 1) (layer "B.Cu") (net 1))
 (segment (start 136.2 92.95) (end 136.6 92.55) (width 1) (layer "B.Cu") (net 1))
 (segment (start 136.55 73.8) (end 139.9 73.8) (width 1) (layer "F.Cu") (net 3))
 (segment (start 136.55 73.8) (end 130.05 73.8) (width 1) (layer "F.Cu") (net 3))
 (segment (start 139.9 73.8) (end 140.3 74.2) (width 1) (layer "F.Cu") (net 3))
 (segment (start 140.3 74.2) (end 140.3 93.4) (width 1) (layer "F.Cu") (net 3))
 (segment (start 140.3 93.4) (end 141.06 94.16) (width 1) (layer "F.Cu") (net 3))
 (segment (start 141.06 94.16) (end 143.5005 94.16) (width 1) (layer "F.Cu") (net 3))
 (segment (start 146.66 99.24) (end 143.5005 99.24) (width 1) (layer "F.Cu") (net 6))
 (segment (start 147 94.651) (end 147 98.9) (width 1) (layer "F.Cu") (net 6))
 (segment (start 152.301 82.799) (end 156.951 82.799) (width 1) (layer "F.Cu") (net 6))
 (segment (start 152.3 82.8) (end 152.301 82.799) (width 1) (layer "F.Cu") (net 6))
 (segment (start 164.05 73.8) (end 157.55 73.8) (width 1) (layer "F.Cu") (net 6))
 (segment (start 146.8 99) (end 146.85 99.05) (width 1) (layer "F.Cu") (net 6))
 (segment (start 147 98.9) (end 146.85 99.05) (width 1) (layer "F.Cu") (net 6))
 (segment (start 146.85 99.05) (end 146.66 99.24) (width 1) (layer "F.Cu") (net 6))
 (segment (start 157.55 82.2) (end 157.55 73.8) (width 1) (layer "F.Cu") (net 6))
 (segment (start 156.951 82.799) (end 157.55 82.2) (width 1) (layer "F.Cu") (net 6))
 (via (at 147 94.651) (size 1.2) (drill 0.3) (layers "F.Cu" "B.Cu") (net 6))
 (via (at 152.3 82.8) (size 1.2) (drill 0.3) (layers "F.Cu" "B.Cu") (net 6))
 (segment (start 147.249 82.8) (end 147 83.049) (width 1) (layer "B.Cu") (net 6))
 (segment (start 147 83.049) (end 147 94.651) (width 1) (layer "B.Cu") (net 6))
 (segment (start 152.3 82.8) (end 147.249 82.8) (width 1) (layer "B.Cu") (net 6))
 (segment (start 150.3 73.8) (end 143.8 73.8) (width 1) (layer "F.Cu") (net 5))
 (segment (start 154.45 98.8) (end 154.45 113.25) (width 1) (layer "F.Cu") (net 5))
 (segment (start 148.5 116.59) (end 150.059 116.59) (width 1) (layer "F.Cu") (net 5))
 (segment (start 154.45 113.25) (end 154.35 113.35) (width 1) (layer "F.Cu") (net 5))
 (segment (start 150.059 116.59) (end 150.149 116.5) (width 1) (layer "F.Cu") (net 5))
 (segment (start 150.3 73.8) (end 150.3 90.5) (width 1) (layer "F.Cu") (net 5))
 (via (at 150.05 116.5) (size 1.2) (drill 0.3) (layers "F.Cu" "B.Cu") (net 5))
 (via (at 150.2 90.55) (size 1.2) (drill 0.3) (layers "F.Cu" "B.Cu") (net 5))
 (via (at 154.35 113.35) (size 1.2) (drill 0.3) (layers "F.Cu" "B.Cu") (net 5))
 (via (at 154.45 98.8) (size 1.2) (drill 0.3) (layers "F.Cu" "B.Cu") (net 5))
 (segment (start 154.5 94.85) (end 155.4 94.85) (width 1) (layer "B.Cu") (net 5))
 (segment (start 159.45 98.2) (end 158.9 98.75) (width 1) (layer "B.Cu") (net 5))
 (segment (start 154.5 94.85) (end 159.55 94.85) (width 1) (layer "B.Cu") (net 5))
 (segment (start 158.9 98.75) (end 154.5 98.75) (width 1) (layer "B.Cu") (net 5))
 (segment (start 159.701 95.001) (end 159.701 97.949) (width 1) (layer "B.Cu") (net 5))
 (segment (start 150.2 90.55) (end 154.5 94.85) (width 1) (layer "B.Cu") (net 5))
 (segment (start 159.55 94.85) (end 159.701 95.001) (width 1) (layer "B.Cu") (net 5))
 (segment (start 153.75 116.5) (end 154.35 115.9) (width 1) (layer "B.Cu") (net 5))
 (segment (start 154.35 115.9) (end 154.35 113.35) (width 1) (layer "B.Cu") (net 5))
 (segment (start 159.701 97.949) (end 159.45 98.2) (width 1) (layer "B.Cu") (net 5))
 (segment (start 150.05 116.5) (end 153.75 116.5) (width 1) (layer "B.Cu") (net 5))
 (segment (start 137.8375 119.15) (end 134.925 119.15) (width 1) (layer "B.Cu") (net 22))
 (segment (start 134.925 119.15) (end 134.9 119.175) (width 0.6) (layer "B.Cu") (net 22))
 (segment (start 132.75 107.35) (end 132.75 110.525) (width 0.6) (layer "B.Cu") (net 21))
 (segment (start 133.1125 106.9875) (end 132.75 107.35) (width 0.6) (layer "B.Cu") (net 21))
 (segment (start 137.2 106.9875) (end 133.1125 106.9875) (width 0.6) (layer "B.Cu") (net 21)))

